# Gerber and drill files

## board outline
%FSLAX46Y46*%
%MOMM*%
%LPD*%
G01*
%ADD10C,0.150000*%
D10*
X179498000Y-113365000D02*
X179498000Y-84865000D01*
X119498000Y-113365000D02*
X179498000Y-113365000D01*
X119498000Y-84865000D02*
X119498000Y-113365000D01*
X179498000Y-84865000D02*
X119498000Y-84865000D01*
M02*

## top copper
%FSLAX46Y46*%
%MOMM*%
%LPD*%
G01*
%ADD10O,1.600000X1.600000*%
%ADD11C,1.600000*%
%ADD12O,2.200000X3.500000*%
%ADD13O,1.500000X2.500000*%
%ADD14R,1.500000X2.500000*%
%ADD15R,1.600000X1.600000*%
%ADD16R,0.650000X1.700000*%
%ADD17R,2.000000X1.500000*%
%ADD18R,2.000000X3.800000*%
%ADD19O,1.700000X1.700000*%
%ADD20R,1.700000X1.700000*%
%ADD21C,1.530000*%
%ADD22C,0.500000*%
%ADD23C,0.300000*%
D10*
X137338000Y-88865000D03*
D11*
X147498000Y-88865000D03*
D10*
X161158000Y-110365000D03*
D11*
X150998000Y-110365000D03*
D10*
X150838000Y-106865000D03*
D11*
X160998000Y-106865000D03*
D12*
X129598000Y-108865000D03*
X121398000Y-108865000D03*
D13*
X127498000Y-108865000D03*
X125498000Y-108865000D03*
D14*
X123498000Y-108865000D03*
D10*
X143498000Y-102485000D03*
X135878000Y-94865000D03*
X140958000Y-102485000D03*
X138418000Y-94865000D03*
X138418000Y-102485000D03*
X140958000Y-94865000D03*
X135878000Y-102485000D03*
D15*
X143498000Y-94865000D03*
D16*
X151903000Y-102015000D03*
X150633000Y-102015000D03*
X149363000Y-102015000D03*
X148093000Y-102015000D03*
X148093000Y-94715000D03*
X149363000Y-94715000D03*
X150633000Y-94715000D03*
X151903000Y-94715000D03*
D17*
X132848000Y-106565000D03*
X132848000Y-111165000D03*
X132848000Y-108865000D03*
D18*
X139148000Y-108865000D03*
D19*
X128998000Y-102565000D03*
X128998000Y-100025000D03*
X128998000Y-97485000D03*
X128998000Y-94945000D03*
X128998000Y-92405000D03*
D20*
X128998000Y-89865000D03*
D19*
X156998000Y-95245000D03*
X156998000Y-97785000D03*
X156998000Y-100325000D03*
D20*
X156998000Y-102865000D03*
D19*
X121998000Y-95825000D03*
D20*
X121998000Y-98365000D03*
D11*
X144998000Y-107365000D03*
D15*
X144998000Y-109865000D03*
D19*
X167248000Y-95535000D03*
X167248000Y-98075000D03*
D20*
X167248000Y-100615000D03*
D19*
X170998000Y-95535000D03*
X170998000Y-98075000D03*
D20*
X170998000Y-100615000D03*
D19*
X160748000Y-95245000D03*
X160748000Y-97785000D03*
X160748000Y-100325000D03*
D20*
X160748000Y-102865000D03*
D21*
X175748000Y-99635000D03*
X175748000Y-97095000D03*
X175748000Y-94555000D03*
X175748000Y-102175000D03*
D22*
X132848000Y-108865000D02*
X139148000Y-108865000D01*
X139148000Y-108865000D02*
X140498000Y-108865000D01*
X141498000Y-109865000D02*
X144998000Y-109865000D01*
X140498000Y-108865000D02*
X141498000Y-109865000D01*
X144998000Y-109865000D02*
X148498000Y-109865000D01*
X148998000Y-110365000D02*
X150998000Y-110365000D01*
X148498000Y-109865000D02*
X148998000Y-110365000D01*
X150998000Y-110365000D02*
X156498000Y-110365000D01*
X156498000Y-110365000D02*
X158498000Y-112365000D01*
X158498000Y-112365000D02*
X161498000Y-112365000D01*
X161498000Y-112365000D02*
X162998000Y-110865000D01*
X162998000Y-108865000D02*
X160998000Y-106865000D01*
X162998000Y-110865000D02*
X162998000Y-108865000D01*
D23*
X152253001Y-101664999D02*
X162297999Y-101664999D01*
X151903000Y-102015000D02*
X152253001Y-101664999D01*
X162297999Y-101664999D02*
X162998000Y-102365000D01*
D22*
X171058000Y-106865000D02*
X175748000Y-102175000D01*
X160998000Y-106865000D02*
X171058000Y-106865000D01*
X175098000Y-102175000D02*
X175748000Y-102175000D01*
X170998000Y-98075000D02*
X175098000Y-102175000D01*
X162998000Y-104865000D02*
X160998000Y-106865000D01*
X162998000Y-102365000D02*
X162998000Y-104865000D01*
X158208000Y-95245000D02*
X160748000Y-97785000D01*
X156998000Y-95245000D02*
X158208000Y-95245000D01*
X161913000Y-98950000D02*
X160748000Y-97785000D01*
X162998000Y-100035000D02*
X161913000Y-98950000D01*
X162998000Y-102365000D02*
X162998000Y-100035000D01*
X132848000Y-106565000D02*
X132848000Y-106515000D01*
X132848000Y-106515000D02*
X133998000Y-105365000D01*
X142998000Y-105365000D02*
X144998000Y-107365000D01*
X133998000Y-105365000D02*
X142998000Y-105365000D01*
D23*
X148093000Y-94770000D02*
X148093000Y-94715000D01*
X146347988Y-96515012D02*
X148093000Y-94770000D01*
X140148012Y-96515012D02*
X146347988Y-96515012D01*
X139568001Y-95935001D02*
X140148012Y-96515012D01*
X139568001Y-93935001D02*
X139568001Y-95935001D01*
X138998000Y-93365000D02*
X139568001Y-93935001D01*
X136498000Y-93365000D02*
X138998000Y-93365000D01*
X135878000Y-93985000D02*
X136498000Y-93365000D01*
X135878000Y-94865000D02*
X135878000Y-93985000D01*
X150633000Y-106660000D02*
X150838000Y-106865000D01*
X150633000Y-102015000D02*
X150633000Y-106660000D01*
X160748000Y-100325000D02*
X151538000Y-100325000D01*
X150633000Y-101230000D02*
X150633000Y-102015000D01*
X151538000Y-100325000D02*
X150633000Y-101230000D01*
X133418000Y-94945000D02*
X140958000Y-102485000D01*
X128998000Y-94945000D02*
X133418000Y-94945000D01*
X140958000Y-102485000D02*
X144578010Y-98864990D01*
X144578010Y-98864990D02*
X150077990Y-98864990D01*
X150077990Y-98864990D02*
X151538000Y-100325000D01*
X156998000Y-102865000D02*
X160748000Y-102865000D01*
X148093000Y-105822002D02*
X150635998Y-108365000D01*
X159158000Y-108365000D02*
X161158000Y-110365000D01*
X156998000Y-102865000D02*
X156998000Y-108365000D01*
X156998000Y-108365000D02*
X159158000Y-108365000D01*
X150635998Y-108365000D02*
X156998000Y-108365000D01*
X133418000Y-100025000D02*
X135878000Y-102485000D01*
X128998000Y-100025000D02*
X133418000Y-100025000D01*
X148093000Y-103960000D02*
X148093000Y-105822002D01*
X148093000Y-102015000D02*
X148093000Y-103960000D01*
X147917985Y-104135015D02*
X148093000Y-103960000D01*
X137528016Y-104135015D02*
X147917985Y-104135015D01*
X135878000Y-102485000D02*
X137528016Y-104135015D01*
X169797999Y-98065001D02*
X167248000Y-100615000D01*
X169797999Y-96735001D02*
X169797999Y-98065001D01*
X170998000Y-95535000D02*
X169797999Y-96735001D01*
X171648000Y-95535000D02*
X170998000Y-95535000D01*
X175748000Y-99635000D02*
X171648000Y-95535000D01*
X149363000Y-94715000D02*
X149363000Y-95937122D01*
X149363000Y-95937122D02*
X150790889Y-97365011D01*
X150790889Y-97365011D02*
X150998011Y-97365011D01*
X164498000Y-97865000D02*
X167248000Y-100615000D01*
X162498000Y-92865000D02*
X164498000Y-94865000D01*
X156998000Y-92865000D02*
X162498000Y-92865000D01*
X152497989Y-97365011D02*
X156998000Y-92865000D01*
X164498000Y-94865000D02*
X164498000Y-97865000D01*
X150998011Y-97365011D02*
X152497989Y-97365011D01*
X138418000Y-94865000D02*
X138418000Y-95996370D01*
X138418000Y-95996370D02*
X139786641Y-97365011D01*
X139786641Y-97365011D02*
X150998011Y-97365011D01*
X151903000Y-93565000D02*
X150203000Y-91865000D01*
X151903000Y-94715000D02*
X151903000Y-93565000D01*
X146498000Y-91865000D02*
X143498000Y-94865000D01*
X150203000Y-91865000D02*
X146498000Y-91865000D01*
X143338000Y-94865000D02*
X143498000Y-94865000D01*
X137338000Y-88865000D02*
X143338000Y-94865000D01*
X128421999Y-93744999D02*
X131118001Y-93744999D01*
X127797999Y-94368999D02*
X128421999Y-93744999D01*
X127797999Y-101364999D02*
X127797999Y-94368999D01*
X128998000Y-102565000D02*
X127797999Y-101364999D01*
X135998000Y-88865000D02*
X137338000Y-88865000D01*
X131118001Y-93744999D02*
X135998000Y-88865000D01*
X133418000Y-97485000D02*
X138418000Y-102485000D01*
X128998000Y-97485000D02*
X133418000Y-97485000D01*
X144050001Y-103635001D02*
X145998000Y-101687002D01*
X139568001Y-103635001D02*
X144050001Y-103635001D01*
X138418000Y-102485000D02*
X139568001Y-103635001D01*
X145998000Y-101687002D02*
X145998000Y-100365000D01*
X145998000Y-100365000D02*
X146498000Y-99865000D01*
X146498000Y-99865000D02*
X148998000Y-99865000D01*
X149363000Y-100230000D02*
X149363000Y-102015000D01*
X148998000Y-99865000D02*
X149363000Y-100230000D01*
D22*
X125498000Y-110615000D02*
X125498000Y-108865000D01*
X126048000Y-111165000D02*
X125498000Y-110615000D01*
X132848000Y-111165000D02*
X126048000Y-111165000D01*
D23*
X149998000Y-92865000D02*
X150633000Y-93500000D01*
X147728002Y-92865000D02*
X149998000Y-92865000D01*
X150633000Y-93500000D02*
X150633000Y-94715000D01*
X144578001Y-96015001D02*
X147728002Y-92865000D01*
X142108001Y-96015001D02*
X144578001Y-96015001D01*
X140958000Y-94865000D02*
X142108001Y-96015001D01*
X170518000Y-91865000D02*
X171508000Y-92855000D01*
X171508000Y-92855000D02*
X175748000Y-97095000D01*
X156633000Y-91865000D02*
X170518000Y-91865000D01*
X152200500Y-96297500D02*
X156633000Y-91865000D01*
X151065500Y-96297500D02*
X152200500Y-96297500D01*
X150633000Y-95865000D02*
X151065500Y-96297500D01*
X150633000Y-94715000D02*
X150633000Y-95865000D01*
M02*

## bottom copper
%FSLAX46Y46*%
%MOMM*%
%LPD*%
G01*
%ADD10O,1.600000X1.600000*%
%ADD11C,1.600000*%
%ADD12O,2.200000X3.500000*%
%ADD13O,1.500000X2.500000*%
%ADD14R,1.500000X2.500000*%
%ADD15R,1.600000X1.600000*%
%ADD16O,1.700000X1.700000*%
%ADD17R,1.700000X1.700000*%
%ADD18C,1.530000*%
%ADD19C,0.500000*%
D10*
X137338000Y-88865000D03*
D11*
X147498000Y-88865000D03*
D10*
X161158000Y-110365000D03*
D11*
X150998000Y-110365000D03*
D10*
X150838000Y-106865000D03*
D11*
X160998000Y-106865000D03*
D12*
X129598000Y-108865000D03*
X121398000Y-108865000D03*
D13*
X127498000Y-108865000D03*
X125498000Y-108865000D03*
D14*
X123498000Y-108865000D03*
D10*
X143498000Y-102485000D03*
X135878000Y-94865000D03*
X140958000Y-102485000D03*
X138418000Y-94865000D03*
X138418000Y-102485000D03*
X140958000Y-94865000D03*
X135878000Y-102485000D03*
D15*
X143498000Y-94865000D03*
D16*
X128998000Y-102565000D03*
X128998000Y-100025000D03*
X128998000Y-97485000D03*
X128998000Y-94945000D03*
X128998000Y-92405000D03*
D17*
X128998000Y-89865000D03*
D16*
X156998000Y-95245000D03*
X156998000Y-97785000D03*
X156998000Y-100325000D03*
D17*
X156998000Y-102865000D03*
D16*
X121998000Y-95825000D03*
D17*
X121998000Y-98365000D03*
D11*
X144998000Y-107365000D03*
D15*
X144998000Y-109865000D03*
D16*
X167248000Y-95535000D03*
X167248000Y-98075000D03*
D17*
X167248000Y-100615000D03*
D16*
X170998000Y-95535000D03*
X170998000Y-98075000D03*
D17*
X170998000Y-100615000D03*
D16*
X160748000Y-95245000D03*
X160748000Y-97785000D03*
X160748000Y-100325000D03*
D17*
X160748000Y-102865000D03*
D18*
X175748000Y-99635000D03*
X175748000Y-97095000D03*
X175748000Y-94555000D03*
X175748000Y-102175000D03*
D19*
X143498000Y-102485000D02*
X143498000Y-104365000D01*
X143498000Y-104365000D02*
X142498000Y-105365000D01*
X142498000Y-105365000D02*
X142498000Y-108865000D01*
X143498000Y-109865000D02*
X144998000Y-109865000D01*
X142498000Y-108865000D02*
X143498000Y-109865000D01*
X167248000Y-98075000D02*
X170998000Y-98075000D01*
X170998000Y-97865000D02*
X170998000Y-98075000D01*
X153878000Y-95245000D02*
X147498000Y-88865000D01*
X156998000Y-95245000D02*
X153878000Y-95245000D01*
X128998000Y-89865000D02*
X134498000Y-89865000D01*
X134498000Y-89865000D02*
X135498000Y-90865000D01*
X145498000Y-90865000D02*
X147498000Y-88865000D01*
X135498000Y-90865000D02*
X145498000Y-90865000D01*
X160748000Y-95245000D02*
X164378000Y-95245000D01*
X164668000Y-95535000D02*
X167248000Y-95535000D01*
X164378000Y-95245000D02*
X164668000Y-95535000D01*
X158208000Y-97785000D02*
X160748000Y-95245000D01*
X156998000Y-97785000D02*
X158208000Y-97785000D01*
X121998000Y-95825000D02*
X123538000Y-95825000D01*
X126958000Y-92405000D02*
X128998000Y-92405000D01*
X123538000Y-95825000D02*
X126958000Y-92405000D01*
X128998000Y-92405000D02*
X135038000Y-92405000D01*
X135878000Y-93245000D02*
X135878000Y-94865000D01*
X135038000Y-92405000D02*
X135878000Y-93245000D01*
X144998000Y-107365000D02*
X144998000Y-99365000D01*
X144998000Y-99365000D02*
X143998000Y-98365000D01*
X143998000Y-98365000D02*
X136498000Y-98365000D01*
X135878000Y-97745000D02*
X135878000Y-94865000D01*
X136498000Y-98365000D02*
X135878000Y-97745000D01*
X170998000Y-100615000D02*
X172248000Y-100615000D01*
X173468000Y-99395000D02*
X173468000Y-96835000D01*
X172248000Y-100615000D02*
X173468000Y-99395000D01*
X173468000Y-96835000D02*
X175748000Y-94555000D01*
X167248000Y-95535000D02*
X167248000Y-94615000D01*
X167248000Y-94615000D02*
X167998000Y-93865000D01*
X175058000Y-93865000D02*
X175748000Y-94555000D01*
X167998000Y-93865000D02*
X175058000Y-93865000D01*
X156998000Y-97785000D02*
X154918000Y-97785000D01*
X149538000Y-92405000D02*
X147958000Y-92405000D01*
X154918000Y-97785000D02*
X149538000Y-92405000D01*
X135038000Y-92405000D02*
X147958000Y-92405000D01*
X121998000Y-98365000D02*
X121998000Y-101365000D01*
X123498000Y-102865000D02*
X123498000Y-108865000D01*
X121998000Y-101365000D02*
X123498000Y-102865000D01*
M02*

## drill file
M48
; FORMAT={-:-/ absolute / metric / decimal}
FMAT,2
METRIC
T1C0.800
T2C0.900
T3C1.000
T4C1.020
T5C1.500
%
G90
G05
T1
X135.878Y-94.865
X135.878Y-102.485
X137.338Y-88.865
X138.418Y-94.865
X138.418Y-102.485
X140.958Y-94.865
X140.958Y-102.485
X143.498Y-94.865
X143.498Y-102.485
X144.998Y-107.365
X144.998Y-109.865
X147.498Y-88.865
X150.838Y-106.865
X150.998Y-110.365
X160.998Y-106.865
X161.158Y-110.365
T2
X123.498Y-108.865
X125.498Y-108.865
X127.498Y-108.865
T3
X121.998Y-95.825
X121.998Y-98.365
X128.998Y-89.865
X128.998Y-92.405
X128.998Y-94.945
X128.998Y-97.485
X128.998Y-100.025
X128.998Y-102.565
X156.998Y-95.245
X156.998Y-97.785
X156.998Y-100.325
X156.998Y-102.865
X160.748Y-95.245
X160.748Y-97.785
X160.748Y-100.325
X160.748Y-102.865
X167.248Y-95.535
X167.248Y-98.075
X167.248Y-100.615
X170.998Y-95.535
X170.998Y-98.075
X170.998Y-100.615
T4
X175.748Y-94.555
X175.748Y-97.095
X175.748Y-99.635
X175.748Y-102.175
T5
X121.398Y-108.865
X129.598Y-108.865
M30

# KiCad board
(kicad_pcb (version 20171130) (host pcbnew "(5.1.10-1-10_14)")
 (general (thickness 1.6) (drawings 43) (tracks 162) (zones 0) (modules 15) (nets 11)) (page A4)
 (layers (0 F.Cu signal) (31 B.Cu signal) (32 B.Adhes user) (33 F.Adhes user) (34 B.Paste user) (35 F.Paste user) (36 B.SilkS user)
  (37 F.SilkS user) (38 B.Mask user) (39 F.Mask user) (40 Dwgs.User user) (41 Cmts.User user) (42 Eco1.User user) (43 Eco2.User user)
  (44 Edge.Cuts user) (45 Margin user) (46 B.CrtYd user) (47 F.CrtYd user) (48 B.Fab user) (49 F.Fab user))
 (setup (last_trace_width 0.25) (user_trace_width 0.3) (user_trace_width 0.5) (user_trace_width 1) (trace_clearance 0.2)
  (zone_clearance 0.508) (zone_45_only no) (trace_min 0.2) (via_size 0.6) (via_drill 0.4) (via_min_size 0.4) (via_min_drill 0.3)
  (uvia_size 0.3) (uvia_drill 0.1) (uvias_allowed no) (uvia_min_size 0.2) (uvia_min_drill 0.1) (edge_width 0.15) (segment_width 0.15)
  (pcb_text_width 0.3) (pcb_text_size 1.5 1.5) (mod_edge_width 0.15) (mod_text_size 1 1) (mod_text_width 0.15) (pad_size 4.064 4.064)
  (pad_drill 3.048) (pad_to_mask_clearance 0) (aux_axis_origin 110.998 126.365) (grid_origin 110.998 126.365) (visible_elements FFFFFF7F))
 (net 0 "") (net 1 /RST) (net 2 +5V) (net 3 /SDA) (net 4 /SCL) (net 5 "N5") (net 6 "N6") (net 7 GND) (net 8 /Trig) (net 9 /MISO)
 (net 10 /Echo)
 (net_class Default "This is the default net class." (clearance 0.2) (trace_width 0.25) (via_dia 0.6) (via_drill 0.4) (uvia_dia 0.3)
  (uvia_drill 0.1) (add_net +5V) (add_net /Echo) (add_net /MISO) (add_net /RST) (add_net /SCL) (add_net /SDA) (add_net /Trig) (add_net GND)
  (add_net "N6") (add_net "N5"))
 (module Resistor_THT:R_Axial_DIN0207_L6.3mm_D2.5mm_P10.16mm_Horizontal (layer F.Cu) (at 147.498 88.865 180)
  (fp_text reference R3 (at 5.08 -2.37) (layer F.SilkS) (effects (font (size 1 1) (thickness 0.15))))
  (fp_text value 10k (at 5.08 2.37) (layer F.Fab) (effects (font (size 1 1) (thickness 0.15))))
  (pad 2 thru_hole oval (at 10.16 0 180) (size 1.6 1.6) (drill 0.8) (layers *.Cu *.Mask) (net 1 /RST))
  (pad 1 thru_hole circle (at 0 0 180) (size 1.6 1.6) (drill 0.8) (layers *.Cu *.Mask) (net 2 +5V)))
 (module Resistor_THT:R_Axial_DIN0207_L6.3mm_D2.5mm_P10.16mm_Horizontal (layer F.Cu) (at 150.998 110.365)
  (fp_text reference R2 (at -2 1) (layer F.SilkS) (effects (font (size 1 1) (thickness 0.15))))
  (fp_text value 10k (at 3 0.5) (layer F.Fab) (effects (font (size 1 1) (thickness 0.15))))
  (pad 2 thru_hole oval (at 10.16 0) (size 1.6 1.6) (drill 0.8) (layers *.Cu *.Mask) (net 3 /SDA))
  (pad 1 thru_hole circle (at 0 0) (size 1.6 1.6) (drill 0.8) (layers *.Cu *.Mask) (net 2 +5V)))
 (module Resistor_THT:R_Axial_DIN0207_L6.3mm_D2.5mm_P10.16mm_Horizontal (layer F.Cu) (at 160.998 106.865 180)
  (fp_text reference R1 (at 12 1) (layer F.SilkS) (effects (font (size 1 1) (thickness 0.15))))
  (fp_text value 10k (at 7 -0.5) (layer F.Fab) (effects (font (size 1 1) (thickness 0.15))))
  (pad 2 thru_hole oval (at 10.16 0 180) (size 1.6 1.6) (drill 0.8) (layers *.Cu *.Mask) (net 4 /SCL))
  (pad 1 thru_hole circle (at 0 0 180) (size 1.6 1.6) (drill 0.8) (layers *.Cu *.Mask) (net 2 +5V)))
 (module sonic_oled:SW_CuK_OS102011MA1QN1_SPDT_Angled (layer F.Cu) (at 123.498 108.865)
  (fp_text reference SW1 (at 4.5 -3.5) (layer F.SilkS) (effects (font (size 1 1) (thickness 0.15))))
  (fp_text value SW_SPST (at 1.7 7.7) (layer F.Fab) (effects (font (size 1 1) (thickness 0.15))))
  (pad "" thru_hole oval (at 6.1 0) (size 2.2 3.5) (drill 1.5) (layers *.Cu *.Mask))
  (pad "" thru_hole oval (at -2.1 0) (size 2.2 3.5) (drill 1.5) (layers *.Cu *.Mask))
  (pad 3 thru_hole oval (at 4 0) (size 1.5 2.5) (drill 0.9) (layers *.Cu *.Mask))
  (pad 2 thru_hole oval (at 2 0) (size 1.5 2.5) (drill 0.9) (layers *.Cu *.Mask) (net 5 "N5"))
  (pad 1 thru_hole rect (at 0 0) (size 1.5 2.5) (drill 0.9) (layers *.Cu *.Mask) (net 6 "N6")))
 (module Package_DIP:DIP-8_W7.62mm (layer F.Cu) (at 143.498 94.865 270)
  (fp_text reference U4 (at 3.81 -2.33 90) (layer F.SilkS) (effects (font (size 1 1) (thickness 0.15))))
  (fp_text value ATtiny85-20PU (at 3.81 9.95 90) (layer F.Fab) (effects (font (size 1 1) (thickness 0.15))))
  (pad 8 thru_hole oval (at 7.62 0 270) (size 1.6 1.6) (drill 0.8) (layers *.Cu *.Mask) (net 2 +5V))
  (pad 4 thru_hole oval (at 0 7.62 270) (size 1.6 1.6) (drill 0.8) (layers *.Cu *.Mask) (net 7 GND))
  (pad 7 thru_hole oval (at 7.62 2.54 270) (size 1.6 1.6) (drill 0.8) (layers *.Cu *.Mask) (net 4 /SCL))
  (pad 3 thru_hole oval (at 0 5.08 270) (size 1.6 1.6) (drill 0.8) (layers *.Cu *.Mask) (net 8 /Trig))
  (pad 6 thru_hole oval (at 7.62 5.08 270) (size 1.6 1.6) (drill 0.8) (layers *.Cu *.Mask) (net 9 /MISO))
  (pad 2 thru_hole oval (at 0 2.54 270) (size 1.6 1.6) (drill 0.8) (layers *.Cu *.Mask) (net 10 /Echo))
  (pad 5 thru_hole oval (at 7.62 7.62 270) (size 1.6 1.6) (drill 0.8) (layers *.Cu *.Mask) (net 3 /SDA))
  (pad 1 thru_hole rect (at 0 0 270) (size 1.6 1.6) (drill 0.8) (layers *.Cu *.Mask) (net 1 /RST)))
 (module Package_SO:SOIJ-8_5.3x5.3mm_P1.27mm (layer F.Cu) (at 149.998 98.365 270)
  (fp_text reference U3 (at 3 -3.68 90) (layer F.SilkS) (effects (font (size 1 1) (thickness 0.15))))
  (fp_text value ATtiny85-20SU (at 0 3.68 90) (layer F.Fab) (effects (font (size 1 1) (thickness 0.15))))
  (pad 8 smd rect (at 3.65 -1.905 270) (size 1.7 0.65) (layers F.Cu F.Paste F.Mask) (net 2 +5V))
  (pad 7 smd rect (at 3.65 -0.635 270) (size 1.7 0.65) (layers F.Cu F.Paste F.Mask) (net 4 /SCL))
  (pad 6 smd rect (at 3.65 0.635 270) (size 1.7 0.65) (layers F.Cu F.Paste F.Mask) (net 9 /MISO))
  (pad 5 smd rect (at 3.65 1.905 270) (size 1.7 0.65) (layers F.Cu F.Paste F.Mask) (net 3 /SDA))
  (pad 4 smd rect (at -3.65 1.905 270) (size 1.7 0.65) (layers F.Cu F.Paste F.Mask) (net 7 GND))
  (pad 3 smd rect (at -3.65 0.635 270) (size 1.7 0.65) (layers F.Cu F.Paste F.Mask) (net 8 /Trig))
  (pad 2 smd rect (at -3.65 -0.635 270) (size 1.7 0.65) (layers F.Cu F.Paste F.Mask) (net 10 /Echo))
  (pad 1 smd rect (at -3.65 -1.905 270) (size 1.7 0.65) (layers F.Cu F.Paste F.Mask) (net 1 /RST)))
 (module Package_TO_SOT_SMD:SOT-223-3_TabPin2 (layer F.Cu) (at 135.998 108.865)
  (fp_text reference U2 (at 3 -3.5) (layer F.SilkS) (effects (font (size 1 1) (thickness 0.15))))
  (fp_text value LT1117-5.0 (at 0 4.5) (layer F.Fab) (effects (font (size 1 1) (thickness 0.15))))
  (pad 1 smd rect (at -3.15 -2.3) (size 2 1.5) (layers F.Cu F.Paste F.Mask) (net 7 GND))
  (pad 3 smd rect (at -3.15 2.3) (size 2 1.5) (layers F.Cu F.Paste F.Mask) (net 5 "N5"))
  (pad 2 smd rect (at -3.15 0) (size 2 1.5) (layers F.Cu F.Paste F.Mask) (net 2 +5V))
  (pad 2 smd rect (at 3.15 0) (size 2 3.8) (layers F.Cu F.Paste F.Mask) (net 2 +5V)))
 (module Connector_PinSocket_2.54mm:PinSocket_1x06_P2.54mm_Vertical (layer F.Cu) (at 128.998 89.865)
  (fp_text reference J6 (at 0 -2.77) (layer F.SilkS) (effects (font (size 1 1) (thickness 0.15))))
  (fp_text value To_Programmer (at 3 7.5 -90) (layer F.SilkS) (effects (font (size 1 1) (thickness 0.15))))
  (pad 6 thru_hole oval (at 0 12.7) (size 1.7 1.7) (drill 1) (layers *.Cu *.Mask) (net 1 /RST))
  (pad 5 thru_hole oval (at 0 10.16) (size 1.7 1.7) (drill 1) (layers *.Cu *.Mask) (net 3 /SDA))
  (pad 4 thru_hole oval (at 0 7.62) (size 1.7 1.7) (drill 1) (layers *.Cu *.Mask) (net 9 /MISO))
  (pad 3 thru_hole oval (at 0 5.08) (size 1.7 1.7) (drill 1) (layers *.Cu *.Mask) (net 4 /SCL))
  (pad 2 thru_hole oval (at 0 2.54) (size 1.7 1.7) (drill 1) (layers *.Cu *.Mask) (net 7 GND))
  (pad 1 thru_hole rect (at 0 0) (size 1.7 1.7) (drill 1) (layers *.Cu *.Mask) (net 2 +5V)))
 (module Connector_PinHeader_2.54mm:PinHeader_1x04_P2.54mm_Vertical (layer F.Cu) (at 156.998 102.865 180)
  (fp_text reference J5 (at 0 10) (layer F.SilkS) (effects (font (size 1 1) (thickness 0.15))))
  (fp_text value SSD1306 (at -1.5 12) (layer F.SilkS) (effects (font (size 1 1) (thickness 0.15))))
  (pad 4 thru_hole oval (at 0 7.62 180) (size 1.7 1.7) (drill 1) (layers *.Cu *.Mask) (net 2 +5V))
  (pad 3 thru_hole oval (at 0 5.08 180) (size 1.7 1.7) (drill 1) (layers *.Cu *.Mask) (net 7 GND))
  (pad 2 thru_hole oval (at 0 2.54 180) (size 1.7 1.7) (drill 1) (layers *.Cu *.Mask) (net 4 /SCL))
  (pad 1 thru_hole rect (at 0 0 180) (size 1.7 1.7) (drill 1) (layers *.Cu *.Mask) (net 3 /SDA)))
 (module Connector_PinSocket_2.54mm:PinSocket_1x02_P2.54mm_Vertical (layer F.Cu) (at 121.998 98.365 180)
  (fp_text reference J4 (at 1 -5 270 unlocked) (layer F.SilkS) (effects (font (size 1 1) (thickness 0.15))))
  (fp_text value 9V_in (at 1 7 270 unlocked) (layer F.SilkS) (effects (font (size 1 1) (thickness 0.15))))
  (pad 2 thru_hole oval (at 0 2.54 180) (size 1.7 1.7) (drill 1) (layers *.Cu *.Mask) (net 7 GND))
  (pad 1 thru_hole rect (at 0 0 180) (size 1.7 1.7) (drill 1) (layers *.Cu *.Mask) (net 6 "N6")))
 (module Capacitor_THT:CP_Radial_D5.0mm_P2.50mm (layer F.Cu) (at 144.998 109.865 90)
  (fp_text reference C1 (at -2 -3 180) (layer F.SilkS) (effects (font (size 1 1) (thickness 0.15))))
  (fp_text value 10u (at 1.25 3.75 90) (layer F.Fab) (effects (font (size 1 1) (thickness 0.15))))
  (pad 2 thru_hole circle (at 2.5 0 90) (size 1.6 1.6) (drill 0.8) (layers *.Cu *.Mask) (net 7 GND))
  (pad 1 thru_hole rect (at 0 0 90) (size 1.6 1.6) (drill 0.8) (layers *.Cu *.Mask) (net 2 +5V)))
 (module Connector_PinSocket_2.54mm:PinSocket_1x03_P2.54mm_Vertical (layer F.Cu) (at 167.248 100.615 180)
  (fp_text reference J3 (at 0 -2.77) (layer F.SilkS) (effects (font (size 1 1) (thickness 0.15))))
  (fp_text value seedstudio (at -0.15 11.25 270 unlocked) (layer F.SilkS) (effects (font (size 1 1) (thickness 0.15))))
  (pad 3 thru_hole oval (at 0 5.08 180) (size 1.7 1.7) (drill 1) (layers *.Cu *.Mask) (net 7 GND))
  (pad 2 thru_hole oval (at 0 2.54 180) (size 1.7 1.7) (drill 1) (layers *.Cu *.Mask) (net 2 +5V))
  (pad 1 thru_hole rect (at 0 0 180) (size 1.7 1.7) (drill 1) (layers *.Cu *.Mask) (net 8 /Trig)))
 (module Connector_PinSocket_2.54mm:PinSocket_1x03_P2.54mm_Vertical (layer F.Cu) (at 170.998 100.615 180)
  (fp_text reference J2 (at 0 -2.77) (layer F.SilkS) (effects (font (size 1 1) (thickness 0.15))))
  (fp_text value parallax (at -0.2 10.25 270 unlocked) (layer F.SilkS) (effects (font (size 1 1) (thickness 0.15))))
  (pad 3 thru_hole oval (at 0 5.08 180) (size 1.7 1.7) (drill 1) (layers *.Cu *.Mask) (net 8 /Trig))
  (pad 2 thru_hole oval (at 0 2.54 180) (size 1.7 1.7) (drill 1) (layers *.Cu *.Mask) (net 2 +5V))
  (pad 1 thru_hole rect (at 0 0 180) (size 1.7 1.7) (drill 1) (layers *.Cu *.Mask) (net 7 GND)))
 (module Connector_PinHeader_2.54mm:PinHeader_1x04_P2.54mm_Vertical (layer F.Cu) (at 160.748 102.865 180)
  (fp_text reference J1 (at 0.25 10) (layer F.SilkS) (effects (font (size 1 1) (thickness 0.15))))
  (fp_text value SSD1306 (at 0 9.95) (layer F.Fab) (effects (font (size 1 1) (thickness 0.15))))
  (pad 4 thru_hole oval (at 0 7.62 180) (size 1.7 1.7) (drill 1) (layers *.Cu *.Mask) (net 7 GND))
  (pad 3 thru_hole oval (at 0 5.08 180) (size 1.7 1.7) (drill 1) (layers *.Cu *.Mask) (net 2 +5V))
  (pad 2 thru_hole oval (at 0 2.54 180) (size 1.7 1.7) (drill 1) (layers *.Cu *.Mask) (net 4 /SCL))
  (pad 1 thru_hole rect (at 0 0 180) (size 1.7 1.7) (drill 1) (layers *.Cu *.Mask) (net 3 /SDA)))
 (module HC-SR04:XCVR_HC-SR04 (layer F.Cu) (at 175.748 98.365 90)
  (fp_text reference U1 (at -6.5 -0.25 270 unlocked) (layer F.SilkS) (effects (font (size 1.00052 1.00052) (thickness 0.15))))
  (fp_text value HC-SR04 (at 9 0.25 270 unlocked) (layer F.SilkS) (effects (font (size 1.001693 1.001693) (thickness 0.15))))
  (pad 2 thru_hole circle (at -1.27 0 90) (size 1.53 1.53) (drill 1.02) (layers *.Cu *.Mask) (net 8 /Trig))
  (pad 3 thru_hole circle (at 1.27 0 90) (size 1.53 1.53) (drill 1.02) (layers *.Cu *.Mask) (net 10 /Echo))
  (pad 4 thru_hole circle (at 3.81 0 90) (size 1.53 1.53) (drill 1.02) (layers *.Cu *.Mask) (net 7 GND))
  (pad 1 thru_hole circle (at -3.81 0 90) (size 1.53 1.53) (drill 1.02) (layers *.Cu *.Mask) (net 2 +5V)))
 (gr_line (start 179.498 113.365) (end 179.498 84.865) (angle 90) (layer Edge.Cuts) (width 0.15))
 (gr_line (start 119.498 113.365) (end 179.498 113.365) (angle 90) (layer Edge.Cuts) (width 0.15))
 (gr_line (start 119.498 84.865) (end 119.498 113.365) (angle 90) (layer Edge.Cuts) (width 0.15))
 (gr_line (start 179.498 84.865) (end 119.498 84.865) (angle 90) (layer Edge.Cuts) (width 0.15))
 (segment (start 132.848 108.865) (end 139.148 108.865) (width 0.5) (layer F.Cu) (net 2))
 (segment (start 139.148 108.865) (end 140.498 108.865) (width 0.5) (layer F.Cu) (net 2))
 (segment (start 141.498 109.865) (end 144.998 109.865) (width 0.5) (layer F.Cu) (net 2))
 (segment (start 140.498 108.865) (end 141.498 109.865) (width 0.5) (layer F.Cu) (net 2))
 (segment (start 144.998 109.865) (end 148.498 109.865) (width 0.5) (layer F.Cu) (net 2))
 (segment (start 148.998 110.365) (end 150.998 110.365) (width 0.5) (layer F.Cu) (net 2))
 (segment (start 148.498 109.865) (end 148.998 110.365) (width 0.5) (layer F.Cu) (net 2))
 (segment (start 150.998 110.365) (end 156.498 110.365) (width 0.5) (layer F.Cu) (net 2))
 (segment (start 156.498 110.365) (end 158.498 112.365) (width 0.5) (layer F.Cu) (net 2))
 (segment (start 158.498 112.365) (end 161.498 112.365) (width 0.5) (layer F.Cu) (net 2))
 (segment (start 161.498 112.365) (end 162.998 110.865) (width 0.5) (layer F.Cu) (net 2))
 (segment (start 162.998 108.865) (end 160.998 106.865) (width 0.5) (layer F.Cu) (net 2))
 (segment (start 162.998 110.865) (end 162.998 108.865) (width 0.5) (layer F.Cu) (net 2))
 (segment (start 143.498 102.485) (end 143.498 104.365) (width 0.5) (layer B.Cu) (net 2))
 (segment (start 143.498 104.365) (end 142.498 105.365) (width 0.5) (layer B.Cu) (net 2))
 (segment (start 142.498 105.365) (end 142.498 108.865) (width 0.5) (layer B.Cu) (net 2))
 (segment (start 143.498 109.865) (end 144.998 109.865) (width 0.5) (layer B.Cu) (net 2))
 (segment (start 142.498 108.865) (end 143.498 109.865) (width 0.5) (layer B.Cu) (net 2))
 (segment (start 152.253001 101.664999) (end 162.297999 101.664999) (width 0.3) (layer F.Cu) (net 2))
 (segment (start 151.903 102.015) (end 152.253001 101.664999) (width 0.3) (layer F.Cu) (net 2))
 (segment (start 162.297999 101.664999) (end 162.998 102.365) (width 0.3) (layer F.Cu) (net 2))
 (segment (start 171.058 106.865) (end 175.748 102.175) (width 0.5) (layer F.Cu) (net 2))
 (segment (start 160.998 106.865) (end 171.058 106.865) (width 0.5) (layer F.Cu) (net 2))
 (segment (start 167.248 98.075) (end 170.998 98.075) (width 0.5) (layer B.Cu) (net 2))
 (segment (start 170.998 97.865) (end 170.998 98.075) (width 0.5) (layer B.Cu) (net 2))
 (segment (start 175.098 102.175) (end 175.748 102.175) (width 0.5) (layer F.Cu) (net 2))
 (segment (start 170.998 98.075) (end 175.098 102.175) (width 0.5) (layer F.Cu) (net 2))
 (segment (start 162.998 104.865) (end 160.998 106.865) (width 0.5) (layer F.Cu) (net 2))
 (segment (start 162.998 102.365) (end 162.998 104.865) (width 0.5) (layer F.Cu) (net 2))
 (segment (start 158.208 95.245) (end 160.748 97.785) (width 0.5) (layer F.Cu) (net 2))
 (segment (start 156.998 95.245) (end 158.208 95.245) (width 0.5) (layer F.Cu) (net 2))
 (segment (start 161.913 98.95) (end 160.748 97.785) (width 0.5) (layer F.Cu) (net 2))
 (segment (start 162.998 100.035) (end 161.913 98.95) (width 0.5) (layer F.Cu) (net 2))
 (segment (start 162.998 102.365) (end 162.998 100.035) (width 0.5) (layer F.Cu) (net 2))
 (segment (start 153.878 95.245) (end 147.498 88.865) (width 0.5) (layer B.Cu) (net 2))
 (segment (start 156.998 95.245) (end 153.878 95.245) (width 0.5) (layer B.Cu) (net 2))
 (segment (start 128.998 89.865) (end 134.498 89.865) (width 0.5) (layer B.Cu) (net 2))
 (segment (start 134.498 89.865) (end 135.498 90.865) (width 0.5) (layer B.Cu) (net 2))
 (segment (start 145.498 90.865) (end 147.498 88.865) (width 0.5) (layer B.Cu) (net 2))
 (segment (start 135.498 90.865) (end 145.498 90.865) (width 0.5) (layer B.Cu) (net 2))
 (segment (start 160.748 95.245) (end 164.378 95.245) (width 0.5) (layer B.Cu) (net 7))
 (segment (start 164.668 95.535) (end 167.248 95.535) (width 0.5) (layer B.Cu) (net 7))
 (segment (start 164.378 95.245) (end 164.668 95.535) (width 0.5) (layer B.Cu) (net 7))
 (segment (start 158.208 97.785) (end 160.748 95.245) (width 0.5) (layer B.Cu) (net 7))
 (segment (start 156.998 97.785) (end 158.208 97.785) (width 0.5) (layer B.Cu) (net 7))
 (segment (start 121.998 95.825) (end 123.538 95.825) (width 0.5) (layer B.Cu) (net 7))
 (segment (start 126.958 92.405) (end 128.998 92.405) (width 0.5) (layer B.Cu) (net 7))
 (segment (start 123.538 95.825) (end 126.958 92.405) (width 0.5) (layer B.Cu) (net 7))
 (segment (start 128.998 92.405) (end 135.038 92.405) (width 0.5) (layer B.Cu) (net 7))
 (segment (start 135.878 93.245) (end 135.878 94.865) (width 0.5) (layer B.Cu) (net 7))
 (segment (start 135.038 92.405) (end 135.878 93.245) (width 0.5) (layer B.Cu) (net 7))
 (segment (start 132.848 106.565) (end 132.848 106.515) (width 0.5) (layer F.Cu) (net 7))
 (segment (start 132.848 106.515) (end 133.998 105.365) (width 0.5) (layer F.Cu) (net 7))
 (segment (start 142.998 105.365) (end 144.998 107.365) (width 0.5) (layer F.Cu) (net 7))
 (segment (start 133.998 105.365) (end 142.998 105.365) (width 0.5) (layer F.Cu) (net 7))
 (segment (start 148.093 94.77) (end 148.093 94.715) (width 0.3) (layer F.Cu) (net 7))
 (segment (start 146.347988 96.515012) (end 148.093 94.77) (width 0.3) (layer F.Cu) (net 7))
 (segment (start 140.148012 96.515012) (end 146.347988 96.515012) (width 0.3) (layer F.Cu) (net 7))
 (segment (start 139.568001 95.935001) (end 140.148012 96.515012) (width 0.3) (layer F.Cu) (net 7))
 (segment (start 139.568001 93.935001) (end 139.568001 95.935001) (width 0.3) (layer F.Cu) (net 7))
 (segment (start 138.998 93.365) (end 139.568001 93.935001) (width 0.3) (layer F.Cu) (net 7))
 (segment (start 136.498 93.365) (end 138.998 93.365) (width 0.3) (layer F.Cu) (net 7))
 (segment (start 135.878 93.985) (end 136.498 93.365) (width 0.3) (layer F.Cu) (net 7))
 (segment (start 135.878 94.865) (end 135.878 93.985) (width 0.3) (layer F.Cu) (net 7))
 (segment (start 144.998 107.365) (end 144.998 99.365) (width 0.5) (layer B.Cu) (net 7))
 (segment (start 144.998 99.365) (end 143.998 98.365) (width 0.5) (layer B.Cu) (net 7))
 (segment (start 143.998 98.365) (end 136.498 98.365) (width 0.5) (layer B.Cu) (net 7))
 (segment (start 135.878 97.745) (end 135.878 94.865) (width 0.5) (layer B.Cu) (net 7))
 (segment (start 136.498 98.365) (end 135.878 97.745) (width 0.5) (layer B.Cu) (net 7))
 (segment (start 170.998 100.615) (end 172.248 100.615) (width 0.5) (layer B.Cu) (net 7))
 (segment (start 173.468 99.395) (end 173.468 96.835) (width 0.5) (layer B.Cu) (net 7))
 (segment (start 172.248 100.615) (end 173.468 99.395) (width 0.5) (layer B.Cu) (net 7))
 (segment (start 173.468 96.835) (end 175.748 94.555) (width 0.5) (layer B.Cu) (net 7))
 (segment (start 167.248 95.535) (end 167.248 94.615) (width 0.5) (layer B.Cu) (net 7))
 (segment (start 167.248 94.615) (end 167.998 93.865) (width 0.5) (layer B.Cu) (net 7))
 (segment (start 175.058 93.865) (end 175.748 94.555) (width 0.5) (layer B.Cu) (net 7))
 (segment (start 167.998 93.865) (end 175.058 93.865) (width 0.5) (layer B.Cu) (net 7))
 (segment (start 156.998 97.785) (end 154.918 97.785) (width 0.5) (layer B.Cu) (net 7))
 (segment (start 149.538 92.405) (end 147.958 92.405) (width 0.5) (layer B.Cu) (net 7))
 (segment (start 154.918 97.785) (end 149.538 92.405) (width 0.5) (layer B.Cu) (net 7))
 (segment (start 135.038 92.405) (end 147.958 92.405) (width 0.5) (layer B.Cu) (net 7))
 (segment (start 150.633 106.66) (end 150.838 106.865) (width 0.3) (layer F.Cu) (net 4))
 (segment (start 150.633 102.015) (end 150.633 106.66) (width 0.3) (layer F.Cu) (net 4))
 (segment (start 160.748 100.325) (end 151.538 100.325) (width 0.3) (layer F.Cu) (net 4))
 (segment (start 150.633 101.23) (end 150.633 102.015) (width 0.3) (layer F.Cu) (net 4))
 (segment (start 151.538 100.325) (end 150.633 101.23) (width 0.3) (layer F.Cu) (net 4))
 (segment (start 133.418 94.945) (end 140.958 102.485) (width 0.3) (layer F.Cu) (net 4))
 (segment (start 128.998 94.945) (end 133.418 94.945) (width 0.3) (layer F.Cu) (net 4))
 (segment (start 140.958 102.485) (end 144.57801 98.86499) (width 0.3) (layer F.Cu) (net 4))
 (segment (start 144.57801 98.86499) (end 150.07799 98.86499) (width 0.3) (layer F.Cu) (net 4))
 (segment (start 150.07799 98.86499) (end 151.538 100.325) (width 0.3) (layer F.Cu) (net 4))
 (segment (start 156.998 102.865) (end 160.748 102.865) (width 0.3) (layer F.Cu) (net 3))
 (segment (start 148.093 105.822002) (end 150.635998 108.365) (width 0.3) (layer F.Cu) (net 3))
 (segment (start 159.158 108.365) (end 161.158 110.365) (width 0.3) (layer F.Cu) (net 3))
 (segment (start 156.998 102.865) (end 156.998 108.365) (width 0.3) (layer F.Cu) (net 3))
 (segment (start 156.998 108.365) (end 159.158 108.365) (width 0.3) (layer F.Cu) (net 3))
 (segment (start 150.635998 108.365) (end 156.998 108.365) (width 0.3) (layer F.Cu) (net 3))
 (segment (start 133.418 100.025) (end 135.878 102.485) (width 0.3) (layer F.Cu) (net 3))
 (segment (start 128.998 100.025) (end 133.418 100.025) (width 0.3) (layer F.Cu) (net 3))
 (segment (start 148.093 103.96) (end 148.093 105.822002) (width 0.3) (layer F.Cu) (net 3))
 (segment (start 148.093 102.015) (end 148.093 103.96) (width 0.3) (layer F.Cu) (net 3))
 (segment (start 147.917985 104.135015) (end 148.093 103.96) (width 0.3) (layer F.Cu) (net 3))
 (segment (start 137.528016 104.135015) (end 147.917985 104.135015) (width 0.3) (layer F.Cu) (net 3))
 (segment (start 135.878 102.485) (end 137.528016 104.135015) (width 0.3) (layer F.Cu) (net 3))
 (segment (start 169.797999 98.065001) (end 167.248 100.615) (width 0.3) (layer F.Cu) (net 8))
 (segment (start 169.797999 96.735001) (end 169.797999 98.065001) (width 0.3) (layer F.Cu) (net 8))
 (segment (start 170.998 95.535) (end 169.797999 96.735001) (width 0.3) (layer F.Cu) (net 8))
 (segment (start 171.648 95.535) (end 170.998 95.535) (width 0.3) (layer F.Cu) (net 8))
 (segment (start 175.748 99.635) (end 171.648 95.535) (width 0.3) (layer F.Cu) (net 8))
 (segment (start 149.363 94.715) (end 149.363 95.937122) (width 0.3) (layer F.Cu) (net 8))
 (segment (start 149.363 95.937122) (end 150.790889 97.365011) (width 0.3) (layer F.Cu) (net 8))
 (segment (start 150.790889 97.365011) (end 150.998011 97.365011) (width 0.3) (layer F.Cu) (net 8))
 (segment (start 164.498 97.865) (end 167.248 100.615) (width 0.3) (layer F.Cu) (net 8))
 (segment (start 162.498 92.865) (end 164.498 94.865) (width 0.3) (layer F.Cu) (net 8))
 (segment (start 156.998 92.865) (end 162.498 92.865) (width 0.3) (layer F.Cu) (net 8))
 (segment (start 152.497989 97.365011) (end 156.998 92.865) (width 0.3) (layer F.Cu) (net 8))
 (segment (start 164.498 94.865) (end 164.498 97.865) (width 0.3) (layer F.Cu) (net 8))
 (segment (start 150.998011 97.365011) (end 152.497989 97.365011) (width 0.3) (layer F.Cu) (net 8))
 (segment (start 138.418 94.865) (end 138.418 95.99637) (width 0.3) (layer F.Cu) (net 8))
 (segment (start 138.418 95.99637) (end 139.786641 97.365011) (width 0.3) (layer F.Cu) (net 8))
 (segment (start 139.786641 97.365011) (end 150.998011 97.365011) (width 0.3) (layer F.Cu) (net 8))
 (segment (start 121.998 98.365) (end 121.998 101.365) (width 0.5) (layer B.Cu) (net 6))
 (segment (start 123.498 102.865) (end 123.498 108.865) (width 0.5) (layer B.Cu) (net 6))
 (segment (start 121.998 101.365) (end 123.498 102.865) (width 0.5) (layer B.Cu) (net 6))
 (segment (start 151.903 93.565) (end 150.203 91.865) (width 0.3) (layer F.Cu) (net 1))
 (segment (start 151.903 94.715) (end 151.903 93.565) (width 0.3) (layer F.Cu) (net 1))
 (segment (start 146.498 91.865) (end 143.498 94.865) (width 0.3) (layer F.Cu) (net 1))
 (segment (start 150.203 91.865) (end 146.498 91.865) (width 0.3) (layer F.Cu) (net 1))
 (segment (start 143.338 94.865) (end 143.498 94.865) (width 0.3) (layer F.Cu) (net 1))
 (segment (start 137.338 88.865) (end 143.338 94.865) (width 0.3) (layer F.Cu) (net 1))
 (segment (start 128.421999 93.744999) (end 131.118001 93.744999) (width 0.3) (layer F.Cu) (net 1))
 (segment (start 127.797999 94.368999) (end 128.421999 93.744999) (width 0.3) (layer F.Cu) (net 1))
 (segment (start 127.797999 101.364999) (end 127.797999 94.368999) (width 0.3) (layer F.Cu) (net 1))
 (segment (start 128.998 102.565) (end 127.797999 101.364999) (width 0.3) (layer F.Cu) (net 1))
 (segment (start 135.998 88.865) (end 137.338 88.865) (width 0.3) (layer F.Cu) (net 1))
 (segment (start 131.118001 93.744999) (end 135.998 88.865) (width 0.3) (layer F.Cu) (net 1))
 (segment (start 133.418 97.485) (end 138.418 102.485) (width 0.3) (layer F.Cu) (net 9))
 (segment (start 128.998 97.485) (end 133.418 97.485) (width 0.3) (layer F.Cu) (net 9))
 (segment (start 144.050001 103.635001) (end 145.998 101.687002) (width 0.3) (layer F.Cu) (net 9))
 (segment (start 139.568001 103.635001) (end 144.050001 103.635001) (width 0.3) (layer F.Cu) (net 9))
 (segment (start 138.418 102.485) (end 139.568001 103.635001) (width 0.3) (layer F.Cu) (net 9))
 (segment (start 145.998 101.687002) (end 145.998 100.365) (width 0.3) (layer F.Cu) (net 9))
 (segment (start 145.998 100.365) (end 146.498 99.865) (width 0.3) (layer F.Cu) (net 9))
 (segment (start 146.498 99.865) (end 148.998 99.865) (width 0.3) (layer F.Cu) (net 9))
 (segment (start 149.363 100.23) (end 149.363 102.015) (width 0.3) (layer F.Cu) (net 9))
 (segment (start 148.998 99.865) (end 149.363 100.23) (width 0.3) (layer F.Cu) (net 9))
 (segment (start 125.498 110.615) (end 125.498 108.865) (width 0.5) (layer F.Cu) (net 5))
 (segment (start 126.048 111.165) (end 125.498 110.615) (width 0.5) (layer F.Cu) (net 5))
 (segment (start 132.848 111.165) (end 126.048 111.165) (width 0.5) (layer F.Cu) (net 5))
 (segment (start 149.998 92.865) (end 150.633 93.5) (width 0.3) (layer F.Cu) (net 10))
 (segment (start 147.728002 92.865) (end 149.998 92.865) (width 0.3) (layer F.Cu) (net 10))
 (segment (start 150.633 93.5) (end 150.633 94.715) (width 0.3) (layer F.Cu) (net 10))
 (segment (start 144.578001 96.015001) (end 147.728002 92.865) (width 0.3) (layer F.Cu) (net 10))
 (segment (start 142.108001 96.015001) (end 144.578001 96.015001) (width 0.3) (layer F.Cu) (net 10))
 (segment (start 140.958 94.865) (end 142.108001 96.015001) (width 0.3) (layer F.Cu) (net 10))
 (segment (start 170.518 91.865) (end 171.508 92.855) (width 0.3) (layer F.Cu) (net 10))
 (segment (start 171.508 92.855) (end 175.748 97.095) (width 0.3) (layer F.Cu) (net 10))
 (segment (start 156.633 91.865) (end 170.518 91.865) (width 0.3) (layer F.Cu) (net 10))
 (segment (start 152.2005 96.2975) (end 156.633 91.865) (width 0.3) (layer F.Cu) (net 10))
 (segment (start 151.0655 96.2975) (end 152.2005 96.2975) (width 0.3) (layer F.Cu) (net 10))
 (segment (start 150.633 95.865) (end 151.0655 96.2975) (width 0.3) (layer F.Cu) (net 10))
 (segment (start 150.633 94.715) (end 150.633 95.865) (width 0.3) (layer F.Cu) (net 10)))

